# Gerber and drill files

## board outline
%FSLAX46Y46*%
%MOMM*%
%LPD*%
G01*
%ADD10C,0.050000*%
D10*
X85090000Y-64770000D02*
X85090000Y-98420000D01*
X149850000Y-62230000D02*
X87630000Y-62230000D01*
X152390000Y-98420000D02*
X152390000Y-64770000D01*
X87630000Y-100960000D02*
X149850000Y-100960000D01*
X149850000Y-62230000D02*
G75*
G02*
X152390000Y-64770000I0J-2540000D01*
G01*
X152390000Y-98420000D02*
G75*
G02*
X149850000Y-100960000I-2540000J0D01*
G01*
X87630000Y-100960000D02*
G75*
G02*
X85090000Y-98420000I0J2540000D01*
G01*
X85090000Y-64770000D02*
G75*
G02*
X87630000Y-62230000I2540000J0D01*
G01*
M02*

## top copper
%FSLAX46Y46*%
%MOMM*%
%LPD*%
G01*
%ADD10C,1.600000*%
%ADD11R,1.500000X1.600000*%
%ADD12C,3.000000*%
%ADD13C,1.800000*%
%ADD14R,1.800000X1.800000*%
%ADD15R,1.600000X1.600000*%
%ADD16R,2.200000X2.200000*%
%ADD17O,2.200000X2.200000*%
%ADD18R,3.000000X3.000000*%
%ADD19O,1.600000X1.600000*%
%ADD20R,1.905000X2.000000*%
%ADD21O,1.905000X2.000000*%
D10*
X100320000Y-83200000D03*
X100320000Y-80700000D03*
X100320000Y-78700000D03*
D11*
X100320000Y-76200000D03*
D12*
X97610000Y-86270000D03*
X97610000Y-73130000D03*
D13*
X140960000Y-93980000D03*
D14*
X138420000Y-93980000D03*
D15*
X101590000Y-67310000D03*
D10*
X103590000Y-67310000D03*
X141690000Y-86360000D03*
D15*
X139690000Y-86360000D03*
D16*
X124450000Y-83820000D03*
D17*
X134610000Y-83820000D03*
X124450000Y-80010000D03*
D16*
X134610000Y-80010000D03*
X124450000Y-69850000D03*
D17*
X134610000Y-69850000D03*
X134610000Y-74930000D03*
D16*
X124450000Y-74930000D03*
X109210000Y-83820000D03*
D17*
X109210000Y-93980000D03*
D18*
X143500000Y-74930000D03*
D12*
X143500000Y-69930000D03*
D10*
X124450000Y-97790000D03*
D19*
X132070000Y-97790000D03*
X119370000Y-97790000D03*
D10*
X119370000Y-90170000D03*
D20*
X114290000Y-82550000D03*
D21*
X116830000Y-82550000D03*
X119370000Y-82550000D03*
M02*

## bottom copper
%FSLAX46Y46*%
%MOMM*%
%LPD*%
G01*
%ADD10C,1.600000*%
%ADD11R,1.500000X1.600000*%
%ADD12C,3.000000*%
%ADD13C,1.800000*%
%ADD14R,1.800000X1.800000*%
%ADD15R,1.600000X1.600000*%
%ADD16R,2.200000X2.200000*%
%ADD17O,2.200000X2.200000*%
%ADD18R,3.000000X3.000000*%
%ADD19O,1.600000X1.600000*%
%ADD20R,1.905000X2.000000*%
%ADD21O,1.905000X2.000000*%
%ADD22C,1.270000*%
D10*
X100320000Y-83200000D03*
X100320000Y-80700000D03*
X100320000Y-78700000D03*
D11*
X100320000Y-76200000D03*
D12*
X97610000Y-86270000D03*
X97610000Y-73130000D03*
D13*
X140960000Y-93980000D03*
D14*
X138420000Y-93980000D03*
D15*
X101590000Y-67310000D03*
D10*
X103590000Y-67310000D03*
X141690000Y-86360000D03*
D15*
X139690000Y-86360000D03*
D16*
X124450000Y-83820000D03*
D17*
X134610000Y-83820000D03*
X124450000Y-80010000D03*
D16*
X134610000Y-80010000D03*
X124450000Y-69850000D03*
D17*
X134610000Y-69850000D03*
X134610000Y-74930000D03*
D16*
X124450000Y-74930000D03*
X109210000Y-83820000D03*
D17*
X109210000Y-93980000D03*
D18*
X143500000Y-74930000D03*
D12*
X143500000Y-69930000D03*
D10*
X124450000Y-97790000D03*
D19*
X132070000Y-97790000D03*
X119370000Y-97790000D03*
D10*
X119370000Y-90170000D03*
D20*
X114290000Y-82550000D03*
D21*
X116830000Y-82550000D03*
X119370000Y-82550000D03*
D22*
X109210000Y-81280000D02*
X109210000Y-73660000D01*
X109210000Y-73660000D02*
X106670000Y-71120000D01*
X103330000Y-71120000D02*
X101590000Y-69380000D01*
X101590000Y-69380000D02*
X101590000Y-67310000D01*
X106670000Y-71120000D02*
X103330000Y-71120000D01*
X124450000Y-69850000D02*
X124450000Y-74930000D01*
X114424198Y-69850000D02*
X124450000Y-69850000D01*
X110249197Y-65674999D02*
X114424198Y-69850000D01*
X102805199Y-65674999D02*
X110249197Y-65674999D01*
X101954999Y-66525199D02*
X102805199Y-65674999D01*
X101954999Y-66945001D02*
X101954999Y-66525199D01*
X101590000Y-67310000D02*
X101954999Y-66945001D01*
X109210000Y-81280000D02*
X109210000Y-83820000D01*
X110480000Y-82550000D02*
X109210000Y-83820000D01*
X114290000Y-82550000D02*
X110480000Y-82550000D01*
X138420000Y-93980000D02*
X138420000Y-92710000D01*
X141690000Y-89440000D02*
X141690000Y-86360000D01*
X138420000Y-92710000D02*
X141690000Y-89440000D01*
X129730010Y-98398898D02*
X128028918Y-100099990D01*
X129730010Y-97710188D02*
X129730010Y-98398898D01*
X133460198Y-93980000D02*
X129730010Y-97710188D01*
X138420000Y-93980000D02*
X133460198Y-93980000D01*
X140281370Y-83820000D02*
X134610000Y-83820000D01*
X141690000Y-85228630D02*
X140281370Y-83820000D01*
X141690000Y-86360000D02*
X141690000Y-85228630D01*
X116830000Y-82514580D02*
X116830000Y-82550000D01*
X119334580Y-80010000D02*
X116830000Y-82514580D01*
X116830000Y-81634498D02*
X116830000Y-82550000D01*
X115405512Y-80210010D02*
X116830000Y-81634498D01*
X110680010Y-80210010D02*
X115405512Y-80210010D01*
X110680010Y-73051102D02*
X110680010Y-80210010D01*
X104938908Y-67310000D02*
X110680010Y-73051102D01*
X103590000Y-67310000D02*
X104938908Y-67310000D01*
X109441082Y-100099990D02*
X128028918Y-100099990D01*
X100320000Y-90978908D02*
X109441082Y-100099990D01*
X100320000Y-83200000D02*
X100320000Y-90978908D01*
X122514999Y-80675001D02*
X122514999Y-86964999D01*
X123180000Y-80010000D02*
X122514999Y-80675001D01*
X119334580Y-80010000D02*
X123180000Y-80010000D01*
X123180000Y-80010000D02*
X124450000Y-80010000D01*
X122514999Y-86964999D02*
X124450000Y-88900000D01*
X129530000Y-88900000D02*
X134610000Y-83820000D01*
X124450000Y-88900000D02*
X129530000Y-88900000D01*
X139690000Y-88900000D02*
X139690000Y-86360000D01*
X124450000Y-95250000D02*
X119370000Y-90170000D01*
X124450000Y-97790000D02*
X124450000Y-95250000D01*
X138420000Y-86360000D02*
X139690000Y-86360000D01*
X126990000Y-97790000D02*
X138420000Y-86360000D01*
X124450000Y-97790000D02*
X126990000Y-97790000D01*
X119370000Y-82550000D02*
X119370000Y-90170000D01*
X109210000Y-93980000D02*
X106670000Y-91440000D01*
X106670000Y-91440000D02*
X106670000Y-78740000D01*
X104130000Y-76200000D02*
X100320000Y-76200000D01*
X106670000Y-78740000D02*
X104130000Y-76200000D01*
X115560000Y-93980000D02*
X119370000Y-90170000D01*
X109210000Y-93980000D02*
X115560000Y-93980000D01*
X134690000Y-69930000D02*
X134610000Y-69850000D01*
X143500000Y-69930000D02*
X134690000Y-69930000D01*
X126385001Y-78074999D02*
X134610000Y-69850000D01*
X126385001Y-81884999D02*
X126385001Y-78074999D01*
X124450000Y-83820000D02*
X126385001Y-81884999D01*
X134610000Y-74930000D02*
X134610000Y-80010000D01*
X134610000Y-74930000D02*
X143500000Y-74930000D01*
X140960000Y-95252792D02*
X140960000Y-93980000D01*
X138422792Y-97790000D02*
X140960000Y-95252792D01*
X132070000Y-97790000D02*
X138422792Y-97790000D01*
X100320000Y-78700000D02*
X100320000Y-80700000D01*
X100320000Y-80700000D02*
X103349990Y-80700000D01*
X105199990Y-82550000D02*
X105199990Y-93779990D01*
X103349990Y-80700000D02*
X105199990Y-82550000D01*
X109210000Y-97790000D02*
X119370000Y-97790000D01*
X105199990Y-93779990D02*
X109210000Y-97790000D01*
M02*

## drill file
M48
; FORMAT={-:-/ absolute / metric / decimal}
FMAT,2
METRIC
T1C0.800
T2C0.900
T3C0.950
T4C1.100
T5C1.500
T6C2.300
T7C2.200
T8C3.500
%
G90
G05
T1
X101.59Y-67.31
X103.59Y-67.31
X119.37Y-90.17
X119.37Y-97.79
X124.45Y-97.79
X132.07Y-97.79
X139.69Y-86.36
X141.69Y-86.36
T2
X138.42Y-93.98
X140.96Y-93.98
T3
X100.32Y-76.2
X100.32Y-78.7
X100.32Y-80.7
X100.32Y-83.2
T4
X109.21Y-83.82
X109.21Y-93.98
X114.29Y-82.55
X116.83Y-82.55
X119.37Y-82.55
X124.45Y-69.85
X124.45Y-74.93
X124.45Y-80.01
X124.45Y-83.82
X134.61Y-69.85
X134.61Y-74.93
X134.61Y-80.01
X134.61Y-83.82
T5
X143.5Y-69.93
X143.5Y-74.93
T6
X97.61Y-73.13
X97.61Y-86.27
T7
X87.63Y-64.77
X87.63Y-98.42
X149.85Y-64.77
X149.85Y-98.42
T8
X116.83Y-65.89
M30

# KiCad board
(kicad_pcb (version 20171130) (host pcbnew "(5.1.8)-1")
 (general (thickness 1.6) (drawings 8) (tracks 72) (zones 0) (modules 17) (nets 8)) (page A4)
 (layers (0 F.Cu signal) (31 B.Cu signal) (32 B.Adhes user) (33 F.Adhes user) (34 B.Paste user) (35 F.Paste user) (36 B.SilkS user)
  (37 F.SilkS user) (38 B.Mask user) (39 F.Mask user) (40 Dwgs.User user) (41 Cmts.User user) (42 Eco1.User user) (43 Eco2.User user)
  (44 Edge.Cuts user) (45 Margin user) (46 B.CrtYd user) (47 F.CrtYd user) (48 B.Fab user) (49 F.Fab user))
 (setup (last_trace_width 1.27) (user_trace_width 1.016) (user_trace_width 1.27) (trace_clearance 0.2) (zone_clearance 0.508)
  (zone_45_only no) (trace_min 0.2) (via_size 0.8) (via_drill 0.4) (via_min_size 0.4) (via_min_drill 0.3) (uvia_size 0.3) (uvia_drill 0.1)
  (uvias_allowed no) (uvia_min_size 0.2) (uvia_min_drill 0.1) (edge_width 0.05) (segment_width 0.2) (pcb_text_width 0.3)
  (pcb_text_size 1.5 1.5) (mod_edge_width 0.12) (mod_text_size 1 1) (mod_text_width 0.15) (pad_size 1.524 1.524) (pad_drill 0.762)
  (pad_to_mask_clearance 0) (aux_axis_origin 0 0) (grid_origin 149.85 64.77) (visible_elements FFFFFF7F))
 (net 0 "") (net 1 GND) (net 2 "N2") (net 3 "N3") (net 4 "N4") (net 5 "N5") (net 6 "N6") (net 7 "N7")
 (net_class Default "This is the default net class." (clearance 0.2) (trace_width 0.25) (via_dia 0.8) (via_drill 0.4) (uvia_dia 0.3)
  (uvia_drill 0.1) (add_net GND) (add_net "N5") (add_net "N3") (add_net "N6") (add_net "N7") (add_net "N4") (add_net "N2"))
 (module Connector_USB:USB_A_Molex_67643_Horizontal (layer F.Cu) (at 100.32 76.2 270)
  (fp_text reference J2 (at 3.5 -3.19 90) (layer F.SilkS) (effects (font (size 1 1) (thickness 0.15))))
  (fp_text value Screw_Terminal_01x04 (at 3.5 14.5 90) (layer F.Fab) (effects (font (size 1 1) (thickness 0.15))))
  (pad 4 thru_hole circle (at 7 0 270) (size 1.6 1.6) (drill 0.95) (layers *.Cu *.Mask) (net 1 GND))
  (pad 3 thru_hole circle (at 4.5 0 270) (size 1.6 1.6) (drill 0.95) (layers *.Cu *.Mask) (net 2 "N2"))
  (pad 2 thru_hole circle (at 2.5 0 270) (size 1.6 1.6) (drill 0.95) (layers *.Cu *.Mask) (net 2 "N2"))
  (pad 1 thru_hole rect (at 0 0 270) (size 1.6 1.5) (drill 0.95) (layers *.Cu *.Mask) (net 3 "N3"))
  (pad 5 thru_hole circle (at 10.07 2.71 270) (size 3 3) (drill 2.3) (layers *.Cu *.Mask))
  (pad 5 thru_hole circle (at -3.07 2.71 270) (size 3 3) (drill 2.3) (layers *.Cu *.Mask)))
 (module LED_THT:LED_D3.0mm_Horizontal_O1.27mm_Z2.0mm (layer F.Cu) (at 138.42 93.98)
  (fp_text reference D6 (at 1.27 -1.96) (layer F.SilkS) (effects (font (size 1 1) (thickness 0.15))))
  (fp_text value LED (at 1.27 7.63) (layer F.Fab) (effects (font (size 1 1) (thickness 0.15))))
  (pad 2 thru_hole circle (at 2.54 0) (size 1.8 1.8) (drill 0.9) (layers *.Cu *.Mask) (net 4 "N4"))
  (pad 1 thru_hole rect (at 0 0) (size 1.8 1.8) (drill 0.9) (layers *.Cu *.Mask) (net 1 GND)))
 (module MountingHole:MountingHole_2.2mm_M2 (layer F.Cu) (at 149.85 98.42)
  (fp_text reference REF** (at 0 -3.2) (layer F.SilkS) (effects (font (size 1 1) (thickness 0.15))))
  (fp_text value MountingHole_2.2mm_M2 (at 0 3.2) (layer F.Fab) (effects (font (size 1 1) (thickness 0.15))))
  (pad 1 np_thru_hole circle (at 0 0) (size 2.2 2.2) (drill 2.2) (layers *.Cu *.Mask)))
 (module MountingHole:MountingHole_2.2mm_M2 (layer F.Cu) (at 87.63 98.42)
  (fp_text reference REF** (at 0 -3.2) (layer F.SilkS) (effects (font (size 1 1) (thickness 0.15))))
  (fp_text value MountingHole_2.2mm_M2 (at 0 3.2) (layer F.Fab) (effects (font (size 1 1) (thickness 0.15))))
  (pad 1 np_thru_hole circle (at 0 0) (size 2.2 2.2) (drill 2.2) (layers *.Cu *.Mask)))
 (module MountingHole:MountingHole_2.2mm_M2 (layer F.Cu) (at 149.85 64.77)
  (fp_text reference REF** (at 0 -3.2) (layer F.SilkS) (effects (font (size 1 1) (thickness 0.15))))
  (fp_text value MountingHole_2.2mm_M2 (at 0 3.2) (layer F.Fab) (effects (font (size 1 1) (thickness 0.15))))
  (pad 1 np_thru_hole circle (at 0 0) (size 2.2 2.2) (drill 2.2) (layers *.Cu *.Mask)))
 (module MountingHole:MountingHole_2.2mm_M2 (layer F.Cu) (at 87.63 64.77)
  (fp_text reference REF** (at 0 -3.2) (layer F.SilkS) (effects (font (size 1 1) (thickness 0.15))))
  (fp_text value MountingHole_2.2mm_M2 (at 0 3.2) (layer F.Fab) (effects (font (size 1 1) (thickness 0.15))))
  (pad 1 np_thru_hole circle (at 0 0) (size 2.2 2.2) (drill 2.2) (layers *.Cu *.Mask)))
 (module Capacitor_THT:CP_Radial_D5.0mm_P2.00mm (layer F.Cu) (at 101.59 67.31)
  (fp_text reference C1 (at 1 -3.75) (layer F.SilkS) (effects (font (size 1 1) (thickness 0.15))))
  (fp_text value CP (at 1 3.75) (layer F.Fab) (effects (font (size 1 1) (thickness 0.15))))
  (pad 1 thru_hole rect (at 0 0) (size 1.6 1.6) (drill 0.8) (layers *.Cu *.Mask) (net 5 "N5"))
  (pad 2 thru_hole circle (at 2 0) (size 1.6 1.6) (drill 0.8) (layers *.Cu *.Mask) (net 1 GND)))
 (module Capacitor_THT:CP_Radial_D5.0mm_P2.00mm (layer F.Cu) (at 139.69 86.36)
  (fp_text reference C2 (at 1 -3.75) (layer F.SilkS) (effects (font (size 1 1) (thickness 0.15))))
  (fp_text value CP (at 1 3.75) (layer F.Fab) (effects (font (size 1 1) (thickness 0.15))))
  (pad 2 thru_hole circle (at 2 0) (size 1.6 1.6) (drill 0.8) (layers *.Cu *.Mask) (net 1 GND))
  (pad 1 thru_hole rect (at 0 0) (size 1.6 1.6) (drill 0.8) (layers *.Cu *.Mask) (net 3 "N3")))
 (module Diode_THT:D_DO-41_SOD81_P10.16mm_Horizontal (layer F.Cu) (at 124.45 83.82)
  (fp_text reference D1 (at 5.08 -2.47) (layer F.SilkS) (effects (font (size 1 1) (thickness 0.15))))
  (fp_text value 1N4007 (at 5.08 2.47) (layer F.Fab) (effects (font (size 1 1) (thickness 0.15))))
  (pad 1 thru_hole rect (at 0 0) (size 2.2 2.2) (drill 1.1) (layers *.Cu *.Mask) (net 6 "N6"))
  (pad 2 thru_hole oval (at 10.16 0) (size 2.2 2.2) (drill 1.1) (layers *.Cu *.Mask) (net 1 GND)))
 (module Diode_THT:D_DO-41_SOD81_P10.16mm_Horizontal (layer F.Cu) (at 134.61 80.01 180)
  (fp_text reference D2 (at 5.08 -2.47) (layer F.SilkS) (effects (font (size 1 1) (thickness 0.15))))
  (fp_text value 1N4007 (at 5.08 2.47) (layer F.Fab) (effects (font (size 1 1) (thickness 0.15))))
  (pad 2 thru_hole oval (at 10.16 0 180) (size 2.2 2.2) (drill 1.1) (layers *.Cu *.Mask) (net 1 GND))
  (pad 1 thru_hole rect (at 0 0 180) (size 2.2 2.2) (drill 1.1) (layers *.Cu *.Mask) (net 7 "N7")))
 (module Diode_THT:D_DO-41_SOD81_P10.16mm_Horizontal (layer F.Cu) (at 124.45 69.85)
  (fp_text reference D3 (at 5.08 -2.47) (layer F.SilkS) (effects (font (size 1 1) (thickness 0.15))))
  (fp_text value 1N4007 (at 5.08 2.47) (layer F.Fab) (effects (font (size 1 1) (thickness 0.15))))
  (pad 1 thru_hole rect (at 0 0) (size 2.2 2.2) (drill 1.1) (layers *.Cu *.Mask) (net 5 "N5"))
  (pad 2 thru_hole oval (at 10.16 0) (size 2.2 2.2) (drill 1.1) (layers *.Cu *.Mask) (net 6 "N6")))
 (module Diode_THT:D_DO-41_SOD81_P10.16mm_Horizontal (layer F.Cu) (at 124.45 74.93)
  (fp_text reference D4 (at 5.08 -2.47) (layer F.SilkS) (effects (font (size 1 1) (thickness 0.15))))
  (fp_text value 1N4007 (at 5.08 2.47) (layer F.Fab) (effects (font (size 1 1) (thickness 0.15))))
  (pad 2 thru_hole oval (at 10.16 0) (size 2.2 2.2) (drill 1.1) (layers *.Cu *.Mask) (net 7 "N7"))
  (pad 1 thru_hole rect (at 0 0) (size 2.2 2.2) (drill 1.1) (layers *.Cu *.Mask) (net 5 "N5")))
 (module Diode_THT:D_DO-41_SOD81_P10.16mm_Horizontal (layer F.Cu) (at 109.21 83.82 270)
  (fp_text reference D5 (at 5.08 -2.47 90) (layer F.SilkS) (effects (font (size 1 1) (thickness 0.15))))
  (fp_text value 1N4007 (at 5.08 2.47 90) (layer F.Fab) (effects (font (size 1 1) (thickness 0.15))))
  (pad 1 thru_hole rect (at 0 0 270) (size 2.2 2.2) (drill 1.1) (layers *.Cu *.Mask) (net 5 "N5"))
  (pad 2 thru_hole oval (at 10.16 0 270) (size 2.2 2.2) (drill 1.1) (layers *.Cu *.Mask) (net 3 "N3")))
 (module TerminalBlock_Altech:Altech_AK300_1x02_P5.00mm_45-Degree (layer F.Cu) (at 143.5 74.93 90)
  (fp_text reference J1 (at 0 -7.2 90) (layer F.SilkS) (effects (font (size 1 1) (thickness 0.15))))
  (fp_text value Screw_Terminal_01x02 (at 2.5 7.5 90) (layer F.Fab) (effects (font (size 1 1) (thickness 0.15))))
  (pad 1 thru_hole rect (at 0 0 90) (size 3 3) (drill 1.5) (layers *.Cu *.Mask) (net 7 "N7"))
  (pad 2 thru_hole circle (at 5 0 90) (size 3 3) (drill 1.5) (layers *.Cu *.Mask) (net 6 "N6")))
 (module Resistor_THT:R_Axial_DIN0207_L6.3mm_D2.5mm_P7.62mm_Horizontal (layer F.Cu) (at 124.45 97.79)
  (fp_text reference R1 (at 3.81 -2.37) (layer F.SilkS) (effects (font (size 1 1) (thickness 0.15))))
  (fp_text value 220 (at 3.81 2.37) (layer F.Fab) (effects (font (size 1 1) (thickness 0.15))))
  (pad 1 thru_hole circle (at 0 0) (size 1.6 1.6) (drill 0.8) (layers *.Cu *.Mask) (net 3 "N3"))
  (pad 2 thru_hole oval (at 7.62 0) (size 1.6 1.6) (drill 0.8) (layers *.Cu *.Mask) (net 4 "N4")))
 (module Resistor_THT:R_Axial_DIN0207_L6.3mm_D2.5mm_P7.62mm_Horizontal (layer F.Cu) (at 119.37 90.17 270)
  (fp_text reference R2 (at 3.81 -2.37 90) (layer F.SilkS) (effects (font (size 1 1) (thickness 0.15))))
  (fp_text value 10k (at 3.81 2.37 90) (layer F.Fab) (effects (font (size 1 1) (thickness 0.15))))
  (pad 2 thru_hole oval (at 7.62 0 270) (size 1.6 1.6) (drill 0.8) (layers *.Cu *.Mask) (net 2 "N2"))
  (pad 1 thru_hole circle (at 0 0 270) (size 1.6 1.6) (drill 0.8) (layers *.Cu *.Mask) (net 3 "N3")))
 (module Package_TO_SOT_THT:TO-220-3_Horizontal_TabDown (layer F.Cu) (at 114.29 82.55)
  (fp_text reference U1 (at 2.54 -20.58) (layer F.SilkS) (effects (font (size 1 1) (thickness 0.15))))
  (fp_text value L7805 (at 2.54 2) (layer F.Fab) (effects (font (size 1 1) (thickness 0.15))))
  (pad "" np_thru_hole oval (at 2.54 -16.66) (size 3.5 3.5) (drill 3.5) (layers *.Cu *.Mask))
  (pad 1 thru_hole rect (at 0 0) (size 1.905 2) (drill 1.1) (layers *.Cu *.Mask) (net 5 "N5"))
  (pad 2 thru_hole oval (at 2.54 0) (size 1.905 2) (drill 1.1) (layers *.Cu *.Mask) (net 1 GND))
  (pad 3 thru_hole oval (at 5.08 0) (size 1.905 2) (drill 1.1) (layers *.Cu *.Mask) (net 3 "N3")))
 (gr_line (start 85.09 64.77) (end 85.09 98.42) (layer Edge.Cuts) (width 0.05))
 (gr_line (start 149.85 62.23) (end 87.63 62.23) (layer Edge.Cuts) (width 0.05))
 (gr_line (start 152.39 98.42) (end 152.39 64.77) (layer Edge.Cuts) (width 0.05))
 (gr_line (start 87.63 100.96) (end 149.85 100.96) (layer Edge.Cuts) (width 0.05))
 (gr_arc (start 149.85 64.77) (end 152.39 64.77) (angle -90) (layer Edge.Cuts) (width 0.05))
 (gr_arc (start 149.85 98.42) (end 149.85 100.96) (angle -90) (layer Edge.Cuts) (width 0.05))
 (gr_arc (start 87.63 98.42) (end 85.09 98.42) (angle -90) (layer Edge.Cuts) (width 0.05))
 (gr_arc (start 87.63 64.77) (end 87.63 62.23) (angle -90) (layer Edge.Cuts) (width 0.05))
 (segment (start 109.21 81.28) (end 109.21 73.66) (width 1.27) (layer B.Cu) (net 5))
 (segment (start 109.21 73.66) (end 106.67 71.12) (width 1.27) (layer B.Cu) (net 5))
 (segment (start 103.33 71.12) (end 101.59 69.38) (width 1.27) (layer B.Cu) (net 5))
 (segment (start 101.59 69.38) (end 101.59 67.31) (width 1.27) (layer B.Cu) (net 5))
 (segment (start 106.67 71.12) (end 103.33 71.12) (width 1.27) (layer B.Cu) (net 5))
 (segment (start 124.45 69.85) (end 124.45 74.93) (width 1.27) (layer B.Cu) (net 5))
 (segment (start 114.424198 69.85) (end 124.45 69.85) (width 1.27) (layer B.Cu) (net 5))
 (segment (start 110.249197 65.674999) (end 114.424198 69.85) (width 1.27) (layer B.Cu) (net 5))
 (segment (start 102.805199 65.674999) (end 110.249197 65.674999) (width 1.27) (layer B.Cu) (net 5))
 (segment (start 101.954999 66.525199) (end 102.805199 65.674999) (width 1.27) (layer B.Cu) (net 5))
 (segment (start 101.954999 66.945001) (end 101.954999 66.525199) (width 1.27) (layer B.Cu) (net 5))
 (segment (start 101.59 67.31) (end 101.954999 66.945001) (width 1.27) (layer B.Cu) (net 5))
 (segment (start 109.21 81.28) (end 109.21 83.82) (width 1.27) (layer B.Cu) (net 5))
 (segment (start 110.48 82.55) (end 109.21 83.82) (width 1.27) (layer B.Cu) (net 5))
 (segment (start 114.29 82.55) (end 110.48 82.55) (width 1.27) (layer B.Cu) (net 5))
 (segment (start 138.42 93.98) (end 138.42 92.71) (width 1.27) (layer B.Cu) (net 1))
 (segment (start 141.69 89.44) (end 141.69 86.36) (width 1.27) (layer B.Cu) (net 1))
 (segment (start 138.42 92.71) (end 141.69 89.44) (width 1.27) (layer B.Cu) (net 1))
 (segment (start 129.73001 98.398898) (end 128.028918 100.09999) (width 1.27) (layer B.Cu) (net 1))
 (segment (start 129.73001 97.710188) (end 129.73001 98.398898) (width 1.27) (layer B.Cu) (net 1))
 (segment (start 133.460198 93.98) (end 129.73001 97.710188) (width 1.27) (layer B.Cu) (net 1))
 (segment (start 138.42 93.98) (end 133.460198 93.98) (width 1.27) (layer B.Cu) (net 1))
 (segment (start 140.28137 83.82) (end 134.61 83.82) (width 1.27) (layer B.Cu) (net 1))
 (segment (start 141.69 85.22863) (end 140.28137 83.82) (width 1.27) (layer B.Cu) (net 1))
 (segment (start 141.69 86.36) (end 141.69 85.22863) (width 1.27) (layer B.Cu) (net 1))
 (segment (start 116.83 82.51458) (end 116.83 82.55) (width 1.27) (layer B.Cu) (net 1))
 (segment (start 119.33458 80.01) (end 116.83 82.51458) (width 1.27) (layer B.Cu) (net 1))
 (segment (start 116.83 81.634498) (end 116.83 82.55) (width 1.27) (layer B.Cu) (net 1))
 (segment (start 115.405512 80.21001) (end 116.83 81.634498) (width 1.27) (layer B.Cu) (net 1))
 (segment (start 110.68001 80.21001) (end 115.405512 80.21001) (width 1.27) (layer B.Cu) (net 1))
 (segment (start 110.68001 73.051102) (end 110.68001 80.21001) (width 1.27) (layer B.Cu) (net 1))
 (segment (start 104.938908 67.31) (end 110.68001 73.051102) (width 1.27) (layer B.Cu) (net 1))
 (segment (start 103.59 67.31) (end 104.938908 67.31) (width 1.27) (layer B.Cu) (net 1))
 (segment (start 109.441082 100.09999) (end 128.028918 100.09999) (width 1.27) (layer B.Cu) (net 1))
 (segment (start 100.32 90.978908) (end 109.441082 100.09999) (width 1.27) (layer B.Cu) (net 1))
 (segment (start 100.32 83.2) (end 100.32 90.978908) (width 1.27) (layer B.Cu) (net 1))
 (segment (start 122.514999 80.675001) (end 122.514999 86.964999) (width 1.27) (layer B.Cu) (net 1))
 (segment (start 123.18 80.01) (end 122.514999 80.675001) (width 1.27) (layer B.Cu) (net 1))
 (segment (start 119.33458 80.01) (end 123.18 80.01) (width 1.27) (layer B.Cu) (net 1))
 (segment (start 123.18 80.01) (end 124.45 80.01) (width 1.27) (layer B.Cu) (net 1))
 (segment (start 122.514999 86.964999) (end 124.45 88.9) (width 1.27) (layer B.Cu) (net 1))
 (segment (start 129.53 88.9) (end 134.61 83.82) (width 1.27) (layer B.Cu) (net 1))
 (segment (start 124.45 88.9) (end 129.53 88.9) (width 1.27) (layer B.Cu) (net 1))
 (segment (start 139.69 88.9) (end 139.69 86.36) (width 1.27) (layer B.Cu) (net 3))
 (segment (start 124.45 95.25) (end 119.37 90.17) (width 1.27) (layer B.Cu) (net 3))
 (segment (start 124.45 97.79) (end 124.45 95.25) (width 1.27) (layer B.Cu) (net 3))
 (segment (start 138.42 86.36) (end 139.69 86.36) (width 1.27) (layer B.Cu) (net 3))
 (segment (start 126.99 97.79) (end 138.42 86.36) (width 1.27) (layer B.Cu) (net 3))
 (segment (start 124.45 97.79) (end 126.99 97.79) (width 1.27) (layer B.Cu) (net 3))
 (segment (start 119.37 82.55) (end 119.37 90.17) (width 1.27) (layer B.Cu) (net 3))
 (segment (start 109.21 93.98) (end 106.67 91.44) (width 1.27) (layer B.Cu) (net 3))
 (segment (start 106.67 91.44) (end 106.67 78.74) (width 1.27) (layer B.Cu) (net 3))
 (segment (start 104.13 76.2) (end 100.32 76.2) (width 1.27) (layer B.Cu) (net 3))
 (segment (start 106.67 78.74) (end 104.13 76.2) (width 1.27) (layer B.Cu) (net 3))
 (segment (start 115.56 93.98) (end 119.37 90.17) (width 1.27) (layer B.Cu) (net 3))
 (segment (start 109.21 93.98) (end 115.56 93.98) (width 1.27) (layer B.Cu) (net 3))
 (segment (start 134.69 69.93) (end 134.61 69.85) (width 1.27) (layer B.Cu) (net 6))
 (segment (start 143.5 69.93) (end 134.69 69.93) (width 1.27) (layer B.Cu) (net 6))
 (segment (start 126.385001 78.074999) (end 134.61 69.85) (width 1.27) (layer B.Cu) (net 6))
 (segment (start 126.385001 81.884999) (end 126.385001 78.074999) (width 1.27) (layer B.Cu) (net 6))
 (segment (start 124.45 83.82) (end 126.385001 81.884999) (width 1.27) (layer B.Cu) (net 6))
 (segment (start 134.61 74.93) (end 134.61 80.01) (width 1.27) (layer B.Cu) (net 7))
 (segment (start 134.61 74.93) (end 143.5 74.93) (width 1.27) (layer B.Cu) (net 7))
 (segment (start 140.96 95.252792) (end 140.96 93.98) (width 1.27) (layer B.Cu) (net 4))
 (segment (start 138.422792 97.79) (end 140.96 95.252792) (width 1.27) (layer B.Cu) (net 4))
 (segment (start 132.07 97.79) (end 138.422792 97.79) (width 1.27) (layer B.Cu) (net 4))
 (segment (start 100.32 78.7) (end 100.32 80.7) (width 1.27) (layer B.Cu) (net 2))
 (segment (start 100.32 80.7) (end 103.34999 80.7) (width 1.27) (layer B.Cu) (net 2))
 (segment (start 105.19999 82.55) (end 105.19999 93.77999) (width 1.27) (layer B.Cu) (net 2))
 (segment (start 103.34999 80.7) (end 105.19999 82.55) (width 1.27) (layer B.Cu) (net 2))
 (segment (start 109.21 97.79) (end 119.37 97.79) (width 1.27) (layer B.Cu) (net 2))
 (segment (start 105.19999 93.77999) (end 109.21 97.79) (width 1.27) (layer B.Cu) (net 2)))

